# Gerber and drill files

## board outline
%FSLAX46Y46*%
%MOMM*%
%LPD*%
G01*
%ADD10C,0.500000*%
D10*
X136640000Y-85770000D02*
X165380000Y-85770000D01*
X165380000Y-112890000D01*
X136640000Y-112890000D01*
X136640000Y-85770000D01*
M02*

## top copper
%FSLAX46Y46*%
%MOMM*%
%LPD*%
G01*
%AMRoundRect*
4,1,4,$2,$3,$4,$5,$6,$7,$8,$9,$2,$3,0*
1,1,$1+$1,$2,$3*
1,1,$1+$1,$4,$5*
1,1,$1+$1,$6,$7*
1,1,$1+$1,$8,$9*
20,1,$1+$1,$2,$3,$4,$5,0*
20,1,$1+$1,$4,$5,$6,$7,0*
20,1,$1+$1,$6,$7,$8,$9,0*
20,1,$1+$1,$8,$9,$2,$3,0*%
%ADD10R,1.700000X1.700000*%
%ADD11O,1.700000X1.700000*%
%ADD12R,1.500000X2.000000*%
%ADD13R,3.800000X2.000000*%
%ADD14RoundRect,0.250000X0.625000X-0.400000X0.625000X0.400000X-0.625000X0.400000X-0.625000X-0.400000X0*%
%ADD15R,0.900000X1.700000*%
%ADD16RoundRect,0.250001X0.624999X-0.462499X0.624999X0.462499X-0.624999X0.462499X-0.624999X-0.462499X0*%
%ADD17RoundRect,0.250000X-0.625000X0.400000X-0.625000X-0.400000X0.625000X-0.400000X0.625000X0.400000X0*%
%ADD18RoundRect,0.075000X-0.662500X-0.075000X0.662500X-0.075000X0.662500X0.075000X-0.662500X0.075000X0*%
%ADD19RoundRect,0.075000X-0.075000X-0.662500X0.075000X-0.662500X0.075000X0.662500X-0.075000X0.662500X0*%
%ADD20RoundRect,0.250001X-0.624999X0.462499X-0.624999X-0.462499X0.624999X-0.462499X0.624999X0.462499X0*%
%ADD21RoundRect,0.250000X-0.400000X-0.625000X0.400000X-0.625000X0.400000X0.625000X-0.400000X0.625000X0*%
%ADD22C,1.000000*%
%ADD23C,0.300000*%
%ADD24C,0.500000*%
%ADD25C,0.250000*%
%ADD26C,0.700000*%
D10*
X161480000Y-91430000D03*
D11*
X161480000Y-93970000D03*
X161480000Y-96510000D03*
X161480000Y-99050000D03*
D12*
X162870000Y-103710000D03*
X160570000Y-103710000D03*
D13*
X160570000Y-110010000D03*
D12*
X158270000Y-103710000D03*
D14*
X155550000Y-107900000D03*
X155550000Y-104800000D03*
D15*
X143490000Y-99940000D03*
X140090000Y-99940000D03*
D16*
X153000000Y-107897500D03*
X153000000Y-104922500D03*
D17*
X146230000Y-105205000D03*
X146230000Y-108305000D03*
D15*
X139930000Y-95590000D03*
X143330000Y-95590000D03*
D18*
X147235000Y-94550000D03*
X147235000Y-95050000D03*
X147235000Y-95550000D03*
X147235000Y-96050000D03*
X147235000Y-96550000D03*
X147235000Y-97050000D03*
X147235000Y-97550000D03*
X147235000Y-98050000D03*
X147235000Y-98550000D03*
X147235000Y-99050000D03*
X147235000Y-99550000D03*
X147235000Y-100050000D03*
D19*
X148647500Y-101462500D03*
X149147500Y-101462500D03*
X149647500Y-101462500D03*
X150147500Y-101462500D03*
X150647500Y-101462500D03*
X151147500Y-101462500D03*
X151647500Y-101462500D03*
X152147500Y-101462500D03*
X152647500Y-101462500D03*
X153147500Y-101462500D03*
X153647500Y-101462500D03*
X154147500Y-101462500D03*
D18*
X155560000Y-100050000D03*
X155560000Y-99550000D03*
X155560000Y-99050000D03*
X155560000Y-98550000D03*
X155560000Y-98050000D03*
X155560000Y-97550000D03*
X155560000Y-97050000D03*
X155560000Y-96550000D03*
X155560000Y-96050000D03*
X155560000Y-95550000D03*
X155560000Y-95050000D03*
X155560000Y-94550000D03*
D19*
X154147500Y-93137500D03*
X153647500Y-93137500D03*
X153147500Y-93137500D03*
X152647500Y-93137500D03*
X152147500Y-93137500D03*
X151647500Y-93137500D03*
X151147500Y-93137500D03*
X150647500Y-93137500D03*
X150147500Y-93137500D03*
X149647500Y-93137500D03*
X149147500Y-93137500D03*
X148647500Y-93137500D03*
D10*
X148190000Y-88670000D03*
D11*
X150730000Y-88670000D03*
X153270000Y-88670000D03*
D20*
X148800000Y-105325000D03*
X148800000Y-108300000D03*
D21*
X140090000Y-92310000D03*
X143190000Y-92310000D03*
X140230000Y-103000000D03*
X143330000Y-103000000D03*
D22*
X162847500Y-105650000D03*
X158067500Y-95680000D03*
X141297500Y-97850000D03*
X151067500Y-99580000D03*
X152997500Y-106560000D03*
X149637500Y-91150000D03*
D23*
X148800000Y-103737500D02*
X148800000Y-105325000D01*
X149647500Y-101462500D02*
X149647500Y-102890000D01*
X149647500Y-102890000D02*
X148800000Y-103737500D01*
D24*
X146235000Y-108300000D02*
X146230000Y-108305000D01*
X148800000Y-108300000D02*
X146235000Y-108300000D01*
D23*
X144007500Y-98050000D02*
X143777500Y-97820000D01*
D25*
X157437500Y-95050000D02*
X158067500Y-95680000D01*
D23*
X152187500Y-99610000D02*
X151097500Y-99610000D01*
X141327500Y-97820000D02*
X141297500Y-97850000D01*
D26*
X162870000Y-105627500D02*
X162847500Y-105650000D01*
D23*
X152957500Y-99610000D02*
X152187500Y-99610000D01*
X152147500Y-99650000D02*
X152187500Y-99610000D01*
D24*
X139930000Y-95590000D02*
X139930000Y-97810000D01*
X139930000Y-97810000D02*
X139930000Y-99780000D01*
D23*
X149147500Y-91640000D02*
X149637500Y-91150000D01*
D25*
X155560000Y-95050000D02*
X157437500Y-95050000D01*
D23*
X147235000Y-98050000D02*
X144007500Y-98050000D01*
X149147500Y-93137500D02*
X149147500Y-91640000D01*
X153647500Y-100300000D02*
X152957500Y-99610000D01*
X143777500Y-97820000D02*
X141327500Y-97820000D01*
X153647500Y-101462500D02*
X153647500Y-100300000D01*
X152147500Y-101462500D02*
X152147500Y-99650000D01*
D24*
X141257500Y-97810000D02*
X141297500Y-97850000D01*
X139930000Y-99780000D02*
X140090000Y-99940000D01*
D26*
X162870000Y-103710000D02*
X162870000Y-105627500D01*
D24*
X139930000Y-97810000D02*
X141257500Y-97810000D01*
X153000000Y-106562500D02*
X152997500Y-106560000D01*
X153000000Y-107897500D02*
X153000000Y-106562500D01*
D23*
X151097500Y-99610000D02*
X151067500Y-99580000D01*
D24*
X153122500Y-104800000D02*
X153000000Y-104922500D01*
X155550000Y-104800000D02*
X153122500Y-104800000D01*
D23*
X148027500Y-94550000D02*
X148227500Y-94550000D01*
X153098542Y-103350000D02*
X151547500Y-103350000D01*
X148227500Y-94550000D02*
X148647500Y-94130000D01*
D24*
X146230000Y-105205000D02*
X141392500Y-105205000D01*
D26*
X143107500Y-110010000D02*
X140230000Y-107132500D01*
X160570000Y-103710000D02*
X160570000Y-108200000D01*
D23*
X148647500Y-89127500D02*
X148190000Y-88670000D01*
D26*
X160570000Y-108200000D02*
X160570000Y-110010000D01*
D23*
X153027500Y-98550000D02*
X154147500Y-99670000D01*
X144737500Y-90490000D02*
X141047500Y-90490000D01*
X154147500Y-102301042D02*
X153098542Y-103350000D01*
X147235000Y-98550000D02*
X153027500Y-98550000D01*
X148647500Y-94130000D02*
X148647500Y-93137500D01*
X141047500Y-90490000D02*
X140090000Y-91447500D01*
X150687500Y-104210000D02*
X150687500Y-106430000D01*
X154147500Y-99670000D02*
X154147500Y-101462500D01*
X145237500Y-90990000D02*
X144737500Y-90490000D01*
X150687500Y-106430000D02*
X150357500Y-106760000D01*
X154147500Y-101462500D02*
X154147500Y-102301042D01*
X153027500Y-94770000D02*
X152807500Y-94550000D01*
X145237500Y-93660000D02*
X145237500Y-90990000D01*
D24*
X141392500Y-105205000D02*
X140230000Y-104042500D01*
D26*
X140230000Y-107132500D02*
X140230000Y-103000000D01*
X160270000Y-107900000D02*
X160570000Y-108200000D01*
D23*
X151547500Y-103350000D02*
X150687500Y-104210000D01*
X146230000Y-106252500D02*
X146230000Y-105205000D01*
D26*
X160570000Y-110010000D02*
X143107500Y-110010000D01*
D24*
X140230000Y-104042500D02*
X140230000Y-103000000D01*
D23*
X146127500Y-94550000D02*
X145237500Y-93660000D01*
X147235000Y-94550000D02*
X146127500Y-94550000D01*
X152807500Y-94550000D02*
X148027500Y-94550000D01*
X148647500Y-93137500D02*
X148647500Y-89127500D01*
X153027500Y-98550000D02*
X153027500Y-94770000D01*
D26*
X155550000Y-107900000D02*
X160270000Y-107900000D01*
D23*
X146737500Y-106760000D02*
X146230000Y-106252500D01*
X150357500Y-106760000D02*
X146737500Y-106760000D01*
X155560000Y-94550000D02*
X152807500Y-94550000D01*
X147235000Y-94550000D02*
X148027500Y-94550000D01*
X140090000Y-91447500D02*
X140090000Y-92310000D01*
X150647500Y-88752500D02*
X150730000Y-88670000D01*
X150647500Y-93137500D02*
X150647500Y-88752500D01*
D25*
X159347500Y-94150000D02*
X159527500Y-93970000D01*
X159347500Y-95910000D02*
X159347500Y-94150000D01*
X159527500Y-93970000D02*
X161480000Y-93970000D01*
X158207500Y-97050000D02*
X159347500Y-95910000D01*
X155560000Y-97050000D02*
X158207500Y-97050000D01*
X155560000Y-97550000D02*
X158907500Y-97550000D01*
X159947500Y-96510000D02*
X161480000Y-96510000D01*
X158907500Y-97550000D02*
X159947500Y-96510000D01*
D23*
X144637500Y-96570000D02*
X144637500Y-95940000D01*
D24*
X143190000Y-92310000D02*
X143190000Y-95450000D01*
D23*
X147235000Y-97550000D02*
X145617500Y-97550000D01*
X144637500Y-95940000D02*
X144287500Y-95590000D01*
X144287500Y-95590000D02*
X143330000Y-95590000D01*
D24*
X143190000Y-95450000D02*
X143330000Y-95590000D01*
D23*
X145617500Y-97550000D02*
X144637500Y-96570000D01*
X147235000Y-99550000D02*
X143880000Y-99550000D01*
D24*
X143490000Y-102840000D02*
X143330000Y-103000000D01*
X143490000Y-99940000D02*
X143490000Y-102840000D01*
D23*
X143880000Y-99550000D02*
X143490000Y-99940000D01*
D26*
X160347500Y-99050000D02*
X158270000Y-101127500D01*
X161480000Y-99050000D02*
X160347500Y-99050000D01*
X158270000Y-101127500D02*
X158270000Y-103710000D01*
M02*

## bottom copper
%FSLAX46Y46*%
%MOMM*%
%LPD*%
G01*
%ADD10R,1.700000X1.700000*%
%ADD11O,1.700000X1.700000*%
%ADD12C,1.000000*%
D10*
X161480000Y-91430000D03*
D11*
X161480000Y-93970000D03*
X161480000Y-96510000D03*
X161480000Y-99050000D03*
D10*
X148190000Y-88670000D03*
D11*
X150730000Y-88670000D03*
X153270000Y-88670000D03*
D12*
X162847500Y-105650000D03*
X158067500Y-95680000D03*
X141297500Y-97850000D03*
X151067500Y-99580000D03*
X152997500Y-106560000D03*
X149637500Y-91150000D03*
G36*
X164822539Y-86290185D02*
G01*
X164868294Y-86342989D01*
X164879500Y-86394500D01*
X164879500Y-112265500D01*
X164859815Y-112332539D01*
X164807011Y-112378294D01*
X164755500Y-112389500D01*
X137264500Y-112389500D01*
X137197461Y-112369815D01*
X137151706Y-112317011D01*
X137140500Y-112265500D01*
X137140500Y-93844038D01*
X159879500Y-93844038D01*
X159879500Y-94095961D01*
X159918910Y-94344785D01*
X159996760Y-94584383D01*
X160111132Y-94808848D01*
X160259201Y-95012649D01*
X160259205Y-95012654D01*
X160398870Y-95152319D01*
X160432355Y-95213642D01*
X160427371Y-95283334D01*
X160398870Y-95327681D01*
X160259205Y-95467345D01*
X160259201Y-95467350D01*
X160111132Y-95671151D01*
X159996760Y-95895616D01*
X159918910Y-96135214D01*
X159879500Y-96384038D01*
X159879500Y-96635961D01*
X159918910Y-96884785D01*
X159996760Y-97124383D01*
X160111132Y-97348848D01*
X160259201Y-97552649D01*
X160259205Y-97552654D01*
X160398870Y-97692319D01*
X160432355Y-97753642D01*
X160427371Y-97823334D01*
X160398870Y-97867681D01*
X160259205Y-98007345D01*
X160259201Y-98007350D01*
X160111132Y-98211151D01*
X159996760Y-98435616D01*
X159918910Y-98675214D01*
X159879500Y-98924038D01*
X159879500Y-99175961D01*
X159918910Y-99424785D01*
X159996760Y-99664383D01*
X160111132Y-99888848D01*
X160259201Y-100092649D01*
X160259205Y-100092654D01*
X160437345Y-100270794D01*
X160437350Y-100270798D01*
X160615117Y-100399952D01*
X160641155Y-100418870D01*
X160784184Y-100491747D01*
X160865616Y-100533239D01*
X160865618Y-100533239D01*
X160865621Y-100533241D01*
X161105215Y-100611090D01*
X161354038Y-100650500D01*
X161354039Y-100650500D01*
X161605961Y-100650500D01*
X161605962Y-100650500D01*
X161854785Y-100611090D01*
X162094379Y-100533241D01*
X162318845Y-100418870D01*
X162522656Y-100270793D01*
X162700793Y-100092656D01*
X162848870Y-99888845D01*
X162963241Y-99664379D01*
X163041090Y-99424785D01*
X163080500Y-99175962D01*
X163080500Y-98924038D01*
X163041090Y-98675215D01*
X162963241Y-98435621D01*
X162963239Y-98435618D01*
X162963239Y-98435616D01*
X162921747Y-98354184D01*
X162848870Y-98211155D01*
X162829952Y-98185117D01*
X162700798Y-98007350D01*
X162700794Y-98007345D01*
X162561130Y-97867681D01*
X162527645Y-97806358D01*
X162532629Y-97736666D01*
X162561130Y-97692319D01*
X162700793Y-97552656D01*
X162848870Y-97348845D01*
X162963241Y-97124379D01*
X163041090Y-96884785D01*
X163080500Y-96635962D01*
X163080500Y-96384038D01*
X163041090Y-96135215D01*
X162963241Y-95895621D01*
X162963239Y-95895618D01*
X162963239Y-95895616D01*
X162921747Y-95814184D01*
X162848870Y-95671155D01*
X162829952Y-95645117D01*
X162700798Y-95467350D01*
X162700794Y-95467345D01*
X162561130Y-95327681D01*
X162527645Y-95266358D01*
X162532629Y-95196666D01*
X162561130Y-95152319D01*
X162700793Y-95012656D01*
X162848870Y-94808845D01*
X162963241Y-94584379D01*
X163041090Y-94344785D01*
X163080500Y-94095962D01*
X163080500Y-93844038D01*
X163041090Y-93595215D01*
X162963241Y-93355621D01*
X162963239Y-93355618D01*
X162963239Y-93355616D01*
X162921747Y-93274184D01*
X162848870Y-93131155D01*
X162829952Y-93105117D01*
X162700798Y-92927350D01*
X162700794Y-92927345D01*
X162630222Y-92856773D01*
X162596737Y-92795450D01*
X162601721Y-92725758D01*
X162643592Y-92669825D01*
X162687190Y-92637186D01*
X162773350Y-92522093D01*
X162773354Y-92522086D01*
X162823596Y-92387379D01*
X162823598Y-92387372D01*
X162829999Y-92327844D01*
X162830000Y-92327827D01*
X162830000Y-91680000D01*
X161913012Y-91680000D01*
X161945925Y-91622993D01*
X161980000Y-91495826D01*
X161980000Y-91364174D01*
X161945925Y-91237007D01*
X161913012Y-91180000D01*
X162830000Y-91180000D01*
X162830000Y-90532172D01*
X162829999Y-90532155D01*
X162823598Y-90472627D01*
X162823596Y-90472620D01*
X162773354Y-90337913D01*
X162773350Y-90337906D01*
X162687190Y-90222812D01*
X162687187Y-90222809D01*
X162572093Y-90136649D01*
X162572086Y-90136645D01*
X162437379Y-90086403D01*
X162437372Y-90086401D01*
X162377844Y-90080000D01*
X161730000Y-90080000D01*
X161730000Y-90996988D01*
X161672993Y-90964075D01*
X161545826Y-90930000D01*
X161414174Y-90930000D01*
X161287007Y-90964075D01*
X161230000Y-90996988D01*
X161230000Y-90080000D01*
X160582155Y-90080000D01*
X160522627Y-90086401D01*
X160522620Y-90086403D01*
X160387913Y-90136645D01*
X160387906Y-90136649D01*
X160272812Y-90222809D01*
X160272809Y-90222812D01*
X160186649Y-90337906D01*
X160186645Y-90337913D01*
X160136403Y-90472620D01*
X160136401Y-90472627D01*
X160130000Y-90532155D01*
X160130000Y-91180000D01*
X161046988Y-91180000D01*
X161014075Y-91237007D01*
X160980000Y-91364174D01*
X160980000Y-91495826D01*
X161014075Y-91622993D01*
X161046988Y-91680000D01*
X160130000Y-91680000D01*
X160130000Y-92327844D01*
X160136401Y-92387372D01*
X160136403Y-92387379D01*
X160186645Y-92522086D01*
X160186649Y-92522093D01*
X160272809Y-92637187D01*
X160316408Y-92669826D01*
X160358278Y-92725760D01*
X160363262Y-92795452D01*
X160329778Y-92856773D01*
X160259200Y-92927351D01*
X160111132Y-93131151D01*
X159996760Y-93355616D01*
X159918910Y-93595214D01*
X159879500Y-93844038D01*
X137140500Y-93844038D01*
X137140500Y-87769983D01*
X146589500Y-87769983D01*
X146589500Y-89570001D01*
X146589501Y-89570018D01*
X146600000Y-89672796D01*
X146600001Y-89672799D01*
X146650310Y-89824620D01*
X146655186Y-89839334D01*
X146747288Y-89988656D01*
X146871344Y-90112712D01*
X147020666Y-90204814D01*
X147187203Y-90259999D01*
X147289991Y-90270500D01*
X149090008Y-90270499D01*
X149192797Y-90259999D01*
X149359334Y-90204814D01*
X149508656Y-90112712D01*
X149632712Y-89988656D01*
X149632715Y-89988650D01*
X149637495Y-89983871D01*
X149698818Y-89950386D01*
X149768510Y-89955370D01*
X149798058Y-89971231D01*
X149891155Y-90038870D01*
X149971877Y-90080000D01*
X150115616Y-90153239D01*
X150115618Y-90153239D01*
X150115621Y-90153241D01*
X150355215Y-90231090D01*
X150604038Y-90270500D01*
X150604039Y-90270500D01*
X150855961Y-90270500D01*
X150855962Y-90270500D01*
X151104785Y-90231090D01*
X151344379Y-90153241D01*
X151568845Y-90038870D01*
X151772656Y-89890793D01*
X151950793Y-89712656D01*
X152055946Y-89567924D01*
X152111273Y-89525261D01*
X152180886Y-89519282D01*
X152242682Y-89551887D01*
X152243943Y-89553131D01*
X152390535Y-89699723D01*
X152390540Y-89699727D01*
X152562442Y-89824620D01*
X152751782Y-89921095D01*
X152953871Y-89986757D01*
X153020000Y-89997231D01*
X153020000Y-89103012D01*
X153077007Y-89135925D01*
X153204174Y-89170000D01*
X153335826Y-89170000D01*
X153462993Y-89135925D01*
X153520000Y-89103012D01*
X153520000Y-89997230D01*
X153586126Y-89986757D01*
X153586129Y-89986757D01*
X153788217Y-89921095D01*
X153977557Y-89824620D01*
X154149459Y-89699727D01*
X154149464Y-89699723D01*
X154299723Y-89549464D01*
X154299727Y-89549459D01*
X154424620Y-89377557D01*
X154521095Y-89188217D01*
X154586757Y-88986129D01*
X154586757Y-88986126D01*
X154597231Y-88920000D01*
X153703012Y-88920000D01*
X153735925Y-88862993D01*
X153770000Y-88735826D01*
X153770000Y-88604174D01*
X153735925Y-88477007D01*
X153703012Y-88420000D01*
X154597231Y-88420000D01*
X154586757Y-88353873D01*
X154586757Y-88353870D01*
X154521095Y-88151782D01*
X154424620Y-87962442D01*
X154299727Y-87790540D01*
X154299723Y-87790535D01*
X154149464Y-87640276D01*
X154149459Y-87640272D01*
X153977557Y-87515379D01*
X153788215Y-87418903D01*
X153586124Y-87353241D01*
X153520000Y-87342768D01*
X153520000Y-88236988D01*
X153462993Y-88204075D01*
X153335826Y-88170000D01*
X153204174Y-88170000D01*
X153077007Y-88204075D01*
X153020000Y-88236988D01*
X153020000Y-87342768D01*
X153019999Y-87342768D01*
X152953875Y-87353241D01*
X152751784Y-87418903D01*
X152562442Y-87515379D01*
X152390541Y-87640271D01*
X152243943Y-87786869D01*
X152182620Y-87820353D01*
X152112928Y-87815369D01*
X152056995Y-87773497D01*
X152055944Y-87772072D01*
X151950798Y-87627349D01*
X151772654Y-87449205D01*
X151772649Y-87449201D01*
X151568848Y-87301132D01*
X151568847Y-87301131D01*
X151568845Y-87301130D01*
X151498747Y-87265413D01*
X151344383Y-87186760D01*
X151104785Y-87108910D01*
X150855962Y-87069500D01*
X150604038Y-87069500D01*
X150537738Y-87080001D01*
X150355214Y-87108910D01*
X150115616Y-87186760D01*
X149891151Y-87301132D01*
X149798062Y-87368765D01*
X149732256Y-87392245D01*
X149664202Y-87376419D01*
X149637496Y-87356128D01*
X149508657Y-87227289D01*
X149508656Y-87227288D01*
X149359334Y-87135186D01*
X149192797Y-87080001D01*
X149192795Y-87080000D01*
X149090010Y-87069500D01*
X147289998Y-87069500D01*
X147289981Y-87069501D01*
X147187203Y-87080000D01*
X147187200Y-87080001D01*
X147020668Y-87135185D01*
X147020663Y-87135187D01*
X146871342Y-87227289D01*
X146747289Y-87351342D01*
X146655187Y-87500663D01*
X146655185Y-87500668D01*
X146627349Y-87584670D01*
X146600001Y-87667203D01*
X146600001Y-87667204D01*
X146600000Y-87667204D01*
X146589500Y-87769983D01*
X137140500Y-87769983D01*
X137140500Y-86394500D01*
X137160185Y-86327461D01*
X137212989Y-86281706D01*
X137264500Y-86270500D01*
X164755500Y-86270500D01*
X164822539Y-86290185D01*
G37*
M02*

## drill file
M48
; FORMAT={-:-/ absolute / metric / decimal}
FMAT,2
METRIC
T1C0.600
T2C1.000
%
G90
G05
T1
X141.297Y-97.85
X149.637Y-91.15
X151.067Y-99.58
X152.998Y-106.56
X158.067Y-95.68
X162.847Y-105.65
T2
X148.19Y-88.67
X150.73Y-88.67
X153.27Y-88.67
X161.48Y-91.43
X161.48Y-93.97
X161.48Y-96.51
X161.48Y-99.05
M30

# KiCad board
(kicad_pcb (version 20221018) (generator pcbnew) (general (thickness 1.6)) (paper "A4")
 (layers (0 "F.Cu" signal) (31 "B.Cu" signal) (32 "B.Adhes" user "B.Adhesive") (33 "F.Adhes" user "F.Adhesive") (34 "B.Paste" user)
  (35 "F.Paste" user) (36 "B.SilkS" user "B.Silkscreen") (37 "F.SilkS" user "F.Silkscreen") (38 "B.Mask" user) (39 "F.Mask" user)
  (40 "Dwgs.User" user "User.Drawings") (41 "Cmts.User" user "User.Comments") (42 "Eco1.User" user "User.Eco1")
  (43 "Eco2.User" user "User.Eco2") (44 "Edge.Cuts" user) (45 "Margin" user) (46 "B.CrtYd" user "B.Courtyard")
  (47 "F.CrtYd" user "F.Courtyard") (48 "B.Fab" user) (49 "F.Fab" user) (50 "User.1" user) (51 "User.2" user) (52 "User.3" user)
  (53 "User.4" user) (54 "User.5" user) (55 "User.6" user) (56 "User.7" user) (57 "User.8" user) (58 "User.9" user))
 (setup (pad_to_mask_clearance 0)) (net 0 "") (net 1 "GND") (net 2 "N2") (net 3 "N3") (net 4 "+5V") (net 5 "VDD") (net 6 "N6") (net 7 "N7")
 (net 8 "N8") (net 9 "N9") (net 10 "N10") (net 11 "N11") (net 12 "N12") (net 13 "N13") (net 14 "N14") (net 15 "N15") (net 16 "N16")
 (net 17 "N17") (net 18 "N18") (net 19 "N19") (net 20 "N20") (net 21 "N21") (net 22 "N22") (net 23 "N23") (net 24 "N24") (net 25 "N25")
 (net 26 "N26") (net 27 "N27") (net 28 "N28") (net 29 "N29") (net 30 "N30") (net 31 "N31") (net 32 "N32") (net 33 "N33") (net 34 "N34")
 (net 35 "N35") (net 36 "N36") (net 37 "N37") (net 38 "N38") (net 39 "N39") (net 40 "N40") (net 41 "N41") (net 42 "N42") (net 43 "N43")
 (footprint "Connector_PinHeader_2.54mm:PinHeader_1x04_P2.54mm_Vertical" (layer "F.Cu") (at 161.48 91.43)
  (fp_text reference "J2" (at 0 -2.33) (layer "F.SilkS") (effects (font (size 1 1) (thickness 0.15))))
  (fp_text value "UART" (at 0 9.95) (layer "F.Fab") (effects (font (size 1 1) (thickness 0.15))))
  (pad "1" thru_hole rect (at 0 0) (size 1.7 1.7) (drill 1) (layers "*.Cu" "*.Mask") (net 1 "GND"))
  (pad "2" thru_hole oval (at 0 2.54) (size 1.7 1.7) (drill 1) (layers "*.Cu" "*.Mask") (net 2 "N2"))
  (pad "3" thru_hole oval (at 0 5.08) (size 1.7 1.7) (drill 1) (layers "*.Cu" "*.Mask") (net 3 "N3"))
  (pad "4" thru_hole oval (at 0 7.62) (size 1.7 1.7) (drill 1) (layers "*.Cu" "*.Mask") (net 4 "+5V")))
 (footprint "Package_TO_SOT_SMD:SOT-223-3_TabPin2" (layer "F.Cu") (at 160.57 106.86 -90)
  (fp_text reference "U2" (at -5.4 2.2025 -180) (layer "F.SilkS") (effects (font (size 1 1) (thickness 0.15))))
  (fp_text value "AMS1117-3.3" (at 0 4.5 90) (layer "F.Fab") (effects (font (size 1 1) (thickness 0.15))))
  (pad "1" smd rect (at -3.15 -2.3 270) (size 2 1.5) (layers "F.Cu" "F.Paste" "F.Mask") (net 1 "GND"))
  (pad "2" smd rect (at -3.15 0 270) (size 2 1.5) (layers "F.Cu" "F.Paste" "F.Mask") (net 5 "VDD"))
  (pad "2" smd rect (at 3.15 0 270) (size 2 3.8) (layers "F.Cu" "F.Paste" "F.Mask") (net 5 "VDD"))
  (pad "3" smd rect (at -3.15 2.3 270) (size 2 1.5) (layers "F.Cu" "F.Paste" "F.Mask") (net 4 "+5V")))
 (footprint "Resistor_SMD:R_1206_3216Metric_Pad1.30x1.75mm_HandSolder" (layer "F.Cu") (at 155.55 106.35 90)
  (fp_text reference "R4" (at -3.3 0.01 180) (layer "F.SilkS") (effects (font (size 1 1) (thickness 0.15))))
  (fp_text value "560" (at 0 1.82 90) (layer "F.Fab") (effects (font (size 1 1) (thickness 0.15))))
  (pad "1" smd roundrect (at -1.55 0 90) (size 1.3 1.75) (layers "F.Cu" "F.Paste" "F.Mask") (roundrect_rratio 0.1923076923) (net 5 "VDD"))
  (pad "2" smd roundrect (at 1.55 0 90) (size 1.3 1.75) (layers "F.Cu" "F.Paste" "F.Mask") (roundrect_rratio 0.1923076923) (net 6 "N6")))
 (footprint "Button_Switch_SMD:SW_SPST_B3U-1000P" (layer "F.Cu") (at 141.79 99.94 180)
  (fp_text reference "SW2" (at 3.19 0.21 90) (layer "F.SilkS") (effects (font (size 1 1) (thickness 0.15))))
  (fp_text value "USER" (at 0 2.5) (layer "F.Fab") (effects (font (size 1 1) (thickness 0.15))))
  (pad "1" smd rect (at -1.7 0 180) (size 0.9 1.7) (layers "F.Cu" "F.Paste" "F.Mask") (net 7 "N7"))
  (pad "2" smd rect (at 1.7 0 180) (size 0.9 1.7) (layers "F.Cu" "F.Paste" "F.Mask") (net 1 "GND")))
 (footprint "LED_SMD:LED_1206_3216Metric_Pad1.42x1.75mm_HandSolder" (layer "F.Cu") (at 153 106.41 90)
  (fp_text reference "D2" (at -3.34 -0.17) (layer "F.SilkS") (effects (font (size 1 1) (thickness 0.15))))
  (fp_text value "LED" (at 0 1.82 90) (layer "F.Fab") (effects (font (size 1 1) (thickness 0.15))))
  (pad "1" smd roundrect (at -1.4875 0 90) (size 1.425 1.75) (layers "F.Cu" "F.Paste" "F.Mask") (roundrect_rratio 0.1754392982)
   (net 1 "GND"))
  (pad "2" smd roundrect (at 1.4875 0 90) (size 1.425 1.75) (layers "F.Cu" "F.Paste" "F.Mask") (roundrect_rratio 0.1754392982) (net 6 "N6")))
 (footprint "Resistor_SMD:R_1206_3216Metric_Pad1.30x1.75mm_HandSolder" (layer "F.Cu") (at 146.23 106.755 -90)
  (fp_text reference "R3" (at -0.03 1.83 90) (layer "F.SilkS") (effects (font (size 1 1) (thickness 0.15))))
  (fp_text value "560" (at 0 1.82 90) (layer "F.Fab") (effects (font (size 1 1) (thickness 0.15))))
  (pad "1" smd roundrect (at -1.55 0 270) (size 1.3 1.75) (layers "F.Cu" "F.Paste" "F.Mask") (roundrect_rratio 0.1923076923) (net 5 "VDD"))
  (pad "2" smd roundrect (at 1.55 0 270) (size 1.3 1.75) (layers "F.Cu" "F.Paste" "F.Mask") (roundrect_rratio 0.1923076923) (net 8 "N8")))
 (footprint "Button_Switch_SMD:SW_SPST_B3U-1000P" (layer "F.Cu") (at 141.63 95.59)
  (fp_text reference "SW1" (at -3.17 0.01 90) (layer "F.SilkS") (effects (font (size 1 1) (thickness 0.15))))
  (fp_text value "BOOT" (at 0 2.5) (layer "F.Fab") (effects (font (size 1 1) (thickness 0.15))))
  (pad "1" smd rect (at -1.7 0) (size 0.9 1.7) (layers "F.Cu" "F.Paste" "F.Mask") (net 1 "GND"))
  (pad "2" smd rect (at 1.7 0) (size 0.9 1.7) (layers "F.Cu" "F.Paste" "F.Mask") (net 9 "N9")))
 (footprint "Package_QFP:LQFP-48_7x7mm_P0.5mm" (layer "F.Cu") (at 151.3975 97.3)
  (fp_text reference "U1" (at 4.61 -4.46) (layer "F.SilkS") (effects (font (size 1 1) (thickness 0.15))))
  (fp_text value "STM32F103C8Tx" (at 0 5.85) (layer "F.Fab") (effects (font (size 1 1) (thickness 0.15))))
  (pad "1" smd roundrect (at -4.1625 -2.75) (size 1.475 0.3) (layers "F.Cu" "F.Paste" "F.Mask") (roundrect_rratio 0.25) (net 5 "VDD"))
  (pad "2" smd roundrect (at -4.1625 -2.25) (size 1.475 0.3) (layers "F.Cu" "F.Paste" "F.Mask") (roundrect_rratio 0.25) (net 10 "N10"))
  (pad "3" smd roundrect (at -4.1625 -1.75) (size 1.475 0.3) (layers "F.Cu" "F.Paste" "F.Mask") (roundrect_rratio 0.25) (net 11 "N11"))
  (pad "4" smd roundrect (at -4.1625 -1.25) (size 1.475 0.3) (layers "F.Cu" "F.Paste" "F.Mask") (roundrect_rratio 0.25) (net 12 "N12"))
  (pad "5" smd roundrect (at -4.1625 -0.75) (size 1.475 0.3) (layers "F.Cu" "F.Paste" "F.Mask") (roundrect_rratio 0.25) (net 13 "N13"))
  (pad "6" smd roundrect (at -4.1625 -0.25) (size 1.475 0.3) (layers "F.Cu" "F.Paste" "F.Mask") (roundrect_rratio 0.25) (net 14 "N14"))
  (pad "7" smd roundrect (at -4.1625 0.25) (size 1.475 0.3) (layers "F.Cu" "F.Paste" "F.Mask") (roundrect_rratio 0.25) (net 9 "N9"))
  (pad "8" smd roundrect (at -4.1625 0.75) (size 1.475 0.3) (layers "F.Cu" "F.Paste" "F.Mask") (roundrect_rratio 0.25) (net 1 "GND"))
  (pad "9" smd roundrect (at -4.1625 1.25) (size 1.475 0.3) (layers "F.Cu" "F.Paste" "F.Mask") (roundrect_rratio 0.25) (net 5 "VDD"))
  (pad "10" smd roundrect (at -4.1625 1.75) (size 1.475 0.3) (layers "F.Cu" "F.Paste" "F.Mask") (roundrect_rratio 0.25) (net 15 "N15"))
  (pad "11" smd roundrect (at -4.1625 2.25) (size 1.475 0.3) (layers "F.Cu" "F.Paste" "F.Mask") (roundrect_rratio 0.25) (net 7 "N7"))
  (pad "12" smd roundrect (at -4.1625 2.75) (size 1.475 0.3) (layers "F.Cu" "F.Paste" "F.Mask") (roundrect_rratio 0.25) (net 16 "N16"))
  (pad "13" smd roundrect (at -2.75 4.1625) (size 0.3 1.475) (layers "F.Cu" "F.Paste" "F.Mask") (roundrect_rratio 0.25) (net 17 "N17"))
  (pad "14" smd roundrect (at -2.25 4.1625) (size 0.3 1.475) (layers "F.Cu" "F.Paste" "F.Mask") (roundrect_rratio 0.25) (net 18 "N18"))
  (pad "15" smd roundrect (at -1.75 4.1625) (size 0.3 1.475) (layers "F.Cu" "F.Paste" "F.Mask") (roundrect_rratio 0.25) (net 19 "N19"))
  (pad "16" smd roundrect (at -1.25 4.1625) (size 0.3 1.475) (layers "F.Cu" "F.Paste" "F.Mask") (roundrect_rratio 0.25) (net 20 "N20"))
  (pad "17" smd roundrect (at -0.75 4.1625) (size 0.3 1.475) (layers "F.Cu" "F.Paste" "F.Mask") (roundrect_rratio 0.25) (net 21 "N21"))
  (pad "18" smd roundrect (at -0.25 4.1625) (size 0.3 1.475) (layers "F.Cu" "F.Paste" "F.Mask") (roundrect_rratio 0.25) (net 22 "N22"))
  (pad "19" smd roundrect (at 0.25 4.1625) (size 0.3 1.475) (layers "F.Cu" "F.Paste" "F.Mask") (roundrect_rratio 0.25) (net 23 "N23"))
  (pad "20" smd roundrect (at 0.75 4.1625) (size 0.3 1.475) (layers "F.Cu" "F.Paste" "F.Mask") (roundrect_rratio 0.25) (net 1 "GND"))
  (pad "21" smd roundrect (at 1.25 4.1625) (size 0.3 1.475) (layers "F.Cu" "F.Paste" "F.Mask") (roundrect_rratio 0.25) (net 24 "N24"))
  (pad "22" smd roundrect (at 1.75 4.1625) (size 0.3 1.475) (layers "F.Cu" "F.Paste" "F.Mask") (roundrect_rratio 0.25) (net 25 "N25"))
  (pad "23" smd roundrect (at 2.25 4.1625) (size 0.3 1.475) (layers "F.Cu" "F.Paste" "F.Mask") (roundrect_rratio 0.25) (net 1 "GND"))
  (pad "24" smd roundrect (at 2.75 4.1625) (size 0.3 1.475) (layers "F.Cu" "F.Paste" "F.Mask") (roundrect_rratio 0.25) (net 5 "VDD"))
  (pad "25" smd roundrect (at 4.1625 2.75) (size 1.475 0.3) (layers "F.Cu" "F.Paste" "F.Mask") (roundrect_rratio 0.25) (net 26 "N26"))
  (pad "26" smd roundrect (at 4.1625 2.25) (size 1.475 0.3) (layers "F.Cu" "F.Paste" "F.Mask") (roundrect_rratio 0.25) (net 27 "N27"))
  (pad "27" smd roundrect (at 4.1625 1.75) (size 1.475 0.3) (layers "F.Cu" "F.Paste" "F.Mask") (roundrect_rratio 0.25) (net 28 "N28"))
  (pad "28" smd roundrect (at 4.1625 1.25) (size 1.475 0.3) (layers "F.Cu" "F.Paste" "F.Mask") (roundrect_rratio 0.25) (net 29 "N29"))
  (pad "29" smd roundrect (at 4.1625 0.75) (size 1.475 0.3) (layers "F.Cu" "F.Paste" "F.Mask") (roundrect_rratio 0.25) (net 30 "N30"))
  (pad "30" smd roundrect (at 4.1625 0.25) (size 1.475 0.3) (layers "F.Cu" "F.Paste" "F.Mask") (roundrect_rratio 0.25) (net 3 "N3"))
  (pad "31" smd roundrect (at 4.1625 -0.25) (size 1.475 0.3) (layers "F.Cu" "F.Paste" "F.Mask") (roundrect_rratio 0.25) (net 2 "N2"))
  (pad "32" smd roundrect (at 4.1625 -0.75) (size 1.475 0.3) (layers "F.Cu" "F.Paste" "F.Mask") (roundrect_rratio 0.25) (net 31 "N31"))
  (pad "33" smd roundrect (at 4.1625 -1.25) (size 1.475 0.3) (layers "F.Cu" "F.Paste" "F.Mask") (roundrect_rratio 0.25) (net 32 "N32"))
  (pad "34" smd roundrect (at 4.1625 -1.75) (size 1.475 0.3) (layers "F.Cu" "F.Paste" "F.Mask") (roundrect_rratio 0.25) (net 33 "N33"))
  (pad "35" smd roundrect (at 4.1625 -2.25) (size 1.475 0.3) (layers "F.Cu" "F.Paste" "F.Mask") (roundrect_rratio 0.25) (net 1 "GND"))
  (pad "36" smd roundrect (at 4.1625 -2.75) (size 1.475 0.3) (layers "F.Cu" "F.Paste" "F.Mask") (roundrect_rratio 0.25) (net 5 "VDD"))
  (pad "37" smd roundrect (at 2.75 -4.1625) (size 0.3 1.475) (layers "F.Cu" "F.Paste" "F.Mask") (roundrect_rratio 0.25) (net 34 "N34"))
  (pad "38" smd roundrect (at 2.25 -4.1625) (size 0.3 1.475) (layers "F.Cu" "F.Paste" "F.Mask") (roundrect_rratio 0.25) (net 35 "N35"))
  (pad "39" smd roundrect (at 1.75 -4.1625) (size 0.3 1.475) (layers "F.Cu" "F.Paste" "F.Mask") (roundrect_rratio 0.25) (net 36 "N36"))
  (pad "40" smd roundrect (at 1.25 -4.1625) (size 0.3 1.475) (layers "F.Cu" "F.Paste" "F.Mask") (roundrect_rratio 0.25) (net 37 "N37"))
  (pad "41" smd roundrect (at 0.75 -4.1625) (size 0.3 1.475) (layers "F.Cu" "F.Paste" "F.Mask") (roundrect_rratio 0.25) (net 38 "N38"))
  (pad "42" smd roundrect (at 0.25 -4.1625) (size 0.3 1.475) (layers "F.Cu" "F.Paste" "F.Mask") (roundrect_rratio 0.25) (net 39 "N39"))
  (pad "43" smd roundrect (at -0.25 -4.1625) (size 0.3 1.475) (layers "F.Cu" "F.Paste" "F.Mask") (roundrect_rratio 0.25) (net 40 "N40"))
  (pad "44" smd roundrect (at -0.75 -4.1625) (size 0.3 1.475) (layers "F.Cu" "F.Paste" "F.Mask") (roundrect_rratio 0.25) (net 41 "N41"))
  (pad "45" smd roundrect (at -1.25 -4.1625) (size 0.3 1.475) (layers "F.Cu" "F.Paste" "F.Mask") (roundrect_rratio 0.25) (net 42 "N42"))
  (pad "46" smd roundrect (at -1.75 -4.1625) (size 0.3 1.475) (layers "F.Cu" "F.Paste" "F.Mask") (roundrect_rratio 0.25) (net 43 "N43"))
  (pad "47" smd roundrect (at -2.25 -4.1625) (size 0.3 1.475) (layers "F.Cu" "F.Paste" "F.Mask") (roundrect_rratio 0.25) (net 1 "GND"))
  (pad "48" smd roundrect (at -2.75 -4.1625) (size 0.3 1.475) (layers "F.Cu" "F.Paste" "F.Mask") (roundrect_rratio 0.25) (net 5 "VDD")))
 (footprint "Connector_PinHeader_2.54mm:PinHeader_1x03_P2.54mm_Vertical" (layer "F.Cu") (at 148.19 88.67 90)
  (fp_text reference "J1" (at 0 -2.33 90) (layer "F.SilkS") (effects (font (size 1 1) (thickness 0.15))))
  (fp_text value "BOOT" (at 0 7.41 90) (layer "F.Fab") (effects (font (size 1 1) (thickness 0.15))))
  (pad "1" thru_hole rect (at 0 0 90) (size 1.7 1.7) (drill 1) (layers "*.Cu" "*.Mask") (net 5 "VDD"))
  (pad "2" thru_hole oval (at 0 2.54 90) (size 1.7 1.7) (drill 1) (layers "*.Cu" "*.Mask") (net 41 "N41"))
  (pad "3" thru_hole oval (at 0 5.08 90) (size 1.7 1.7) (drill 1) (layers "*.Cu" "*.Mask") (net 1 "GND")))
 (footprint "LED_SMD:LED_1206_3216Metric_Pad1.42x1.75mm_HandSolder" (layer "F.Cu") (at 148.8 106.8125 -90)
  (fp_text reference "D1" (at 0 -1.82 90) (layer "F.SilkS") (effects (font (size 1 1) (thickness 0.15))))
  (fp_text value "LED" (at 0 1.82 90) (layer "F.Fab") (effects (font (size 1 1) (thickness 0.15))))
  (pad "1" smd roundrect (at -1.4875 0 270) (size 1.425 1.75) (layers "F.Cu" "F.Paste" "F.Mask") (roundrect_rratio 0.1754392982)
   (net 19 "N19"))
  (pad "2" smd roundrect (at 1.4875 0 270) (size 1.425 1.75) (layers "F.Cu" "F.Paste" "F.Mask") (roundrect_rratio 0.1754392982) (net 8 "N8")))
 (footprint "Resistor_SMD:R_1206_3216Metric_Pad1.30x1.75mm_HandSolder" (layer "F.Cu") (at 141.64 92.31)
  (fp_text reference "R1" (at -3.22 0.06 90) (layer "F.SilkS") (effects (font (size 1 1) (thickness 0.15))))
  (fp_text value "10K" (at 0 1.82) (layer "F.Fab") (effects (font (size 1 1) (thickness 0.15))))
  (pad "1" smd roundrect (at -1.55 0) (size 1.3 1.75) (layers "F.Cu" "F.Paste" "F.Mask") (roundrect_rratio 0.1923076923) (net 5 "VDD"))
  (pad "2" smd roundrect (at 1.55 0) (size 1.3 1.75) (layers "F.Cu" "F.Paste" "F.Mask") (roundrect_rratio 0.1923076923) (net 9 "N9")))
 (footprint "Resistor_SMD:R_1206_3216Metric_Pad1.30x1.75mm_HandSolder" (layer "F.Cu") (at 141.78 103)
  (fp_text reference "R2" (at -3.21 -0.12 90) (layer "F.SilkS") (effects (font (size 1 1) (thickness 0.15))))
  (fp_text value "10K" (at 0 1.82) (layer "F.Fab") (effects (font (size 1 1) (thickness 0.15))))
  (pad "1" smd roundrect (at -1.55 0) (size 1.3 1.75) (layers "F.Cu" "F.Paste" "F.Mask") (roundrect_rratio 0.1923076923) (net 5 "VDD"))
  (pad "2" smd roundrect (at 1.55 0) (size 1.3 1.75) (layers "F.Cu" "F.Paste" "F.Mask") (roundrect_rratio 0.1923076923) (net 7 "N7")))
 (gr_rect (start 136.64 85.77) (end 165.38 112.89) (stroke (width 0.5) (type default)) (fill none) (layer "Edge.Cuts"))
 (segment (start 148.8 103.7375) (end 148.8 105.325) (width 0.3) (layer "F.Cu") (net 19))
 (segment (start 149.6475 101.4625) (end 149.6475 102.89) (width 0.3) (layer "F.Cu") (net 19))
 (segment (start 149.6475 102.89) (end 148.8 103.7375) (width 0.3) (layer "F.Cu") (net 19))
 (segment (start 146.235 108.3) (end 146.23 108.305) (width 0.5) (layer "F.Cu") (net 8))
 (segment (start 148.8 108.3) (end 146.235 108.3) (width 0.5) (layer "F.Cu") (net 8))
 (segment (start 144.0075 98.05) (end 143.7775 97.82) (width 0.3) (layer "F.Cu") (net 1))
 (segment (start 157.4375 95.05) (end 158.0675 95.68) (width 0.25) (layer "F.Cu") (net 1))
 (segment (start 152.1875 99.61) (end 151.0975 99.61) (width 0.3) (layer "F.Cu") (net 1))
 (segment (start 141.3275 97.82) (end 141.2975 97.85) (width 0.3) (layer "F.Cu") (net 1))
 (segment (start 162.87 105.6275) (end 162.8475 105.65) (width 0.7) (layer "F.Cu") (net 1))
 (segment (start 152.9575 99.61) (end 152.1875 99.61) (width 0.3) (layer "F.Cu") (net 1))
 (segment (start 152.1475 99.65) (end 152.1875 99.61) (width 0.3) (layer "F.Cu") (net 1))
 (segment (start 139.93 95.59) (end 139.93 97.81) (width 0.5) (layer "F.Cu") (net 1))
 (segment (start 139.93 97.81) (end 139.93 99.78) (width 0.5) (layer "F.Cu") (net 1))
 (segment (start 149.1475 91.64) (end 149.6375 91.15) (width 0.3) (layer "F.Cu") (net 1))
 (segment (start 155.56 95.05) (end 157.4375 95.05) (width 0.25) (layer "F.Cu") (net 1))
 (segment (start 147.235 98.05) (end 144.0075 98.05) (width 0.3) (layer "F.Cu") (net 1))
 (segment (start 149.1475 93.1375) (end 149.1475 91.64) (width 0.3) (layer "F.Cu") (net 1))
 (segment (start 153.6475 100.3) (end 152.9575 99.61) (width 0.3) (layer "F.Cu") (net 1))
 (segment (start 143.7775 97.82) (end 141.3275 97.82) (width 0.3) (layer "F.Cu") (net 1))
 (segment (start 153.6475 101.4625) (end 153.6475 100.3) (width 0.3) (layer "F.Cu") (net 1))
 (segment (start 152.1475 101.4625) (end 152.1475 99.65) (width 0.3) (layer "F.Cu") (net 1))
 (segment (start 141.2575 97.81) (end 141.2975 97.85) (width 0.5) (layer "F.Cu") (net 1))
 (segment (start 139.93 99.78) (end 140.09 99.94) (width 0.5) (layer "F.Cu") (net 1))
 (segment (start 162.87 103.71) (end 162.87 105.6275) (width 0.7) (layer "F.Cu") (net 1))
 (segment (start 139.93 97.81) (end 141.2575 97.81) (width 0.5) (layer "F.Cu") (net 1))
 (segment (start 153 106.5625) (end 152.9975 106.56) (width 0.5) (layer "F.Cu") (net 1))
 (segment (start 153 107.8975) (end 153 106.5625) (width 0.5) (layer "F.Cu") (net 1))
 (segment (start 151.0975 99.61) (end 151.0675 99.58) (width 0.3) (layer "F.Cu") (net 1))
 (via (at 162.8475 105.65) (size 1) (drill 0.6) (layers "F.Cu" "B.Cu") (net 1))
 (via (at 158.0675 95.68) (size 1) (drill 0.6) (layers "F.Cu" "B.Cu") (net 1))
 (via (at 141.2975 97.85) (size 1) (drill 0.6) (layers "F.Cu" "B.Cu") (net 1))
 (via (at 151.0675 99.58) (size 1) (drill 0.6) (layers "F.Cu" "B.Cu") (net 1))
 (via (at 152.9975 106.56) (size 1) (drill 0.6) (layers "F.Cu" "B.Cu") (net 1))
 (via (at 149.6375 91.15) (size 1) (drill 0.6) (layers "F.Cu" "B.Cu") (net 1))
 (segment (start 153.1225 104.8) (end 153 104.9225) (width 0.5) (layer "F.Cu") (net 6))
 (segment (start 155.55 104.8) (end 153.1225 104.8) (width 0.5) (layer "F.Cu") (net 6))
 (segment (start 148.0275 94.55) (end 148.2275 94.55) (width 0.3) (layer "F.Cu") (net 5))
 (segment (start 153.098542 103.35) (end 151.5475 103.35) (width 0.3) (layer "F.Cu") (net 5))
 (segment (start 148.2275 94.55) (end 148.6475 94.13) (width 0.3) (layer "F.Cu") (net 5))
 (segment (start 146.23 105.205) (end 141.3925 105.205) (width 0.5) (layer "F.Cu") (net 5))
 (segment (start 143.1075 110.01) (end 140.23 107.1325) (width 0.7) (layer "F.Cu") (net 5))
 (segment (start 160.57 103.71) (end 160.57 108.2) (width 0.7) (layer "F.Cu") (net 5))
 (segment (start 148.6475 89.1275) (end 148.19 88.67) (width 0.3) (layer "F.Cu") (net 5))
 (segment (start 160.57 108.2) (end 160.57 110.01) (width 0.7) (layer "F.Cu") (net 5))
 (segment (start 153.0275 98.55) (end 154.1475 99.67) (width 0.3) (layer "F.Cu") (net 5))
 (segment (start 144.7375 90.49) (end 141.0475 90.49) (width 0.3) (layer "F.Cu") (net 5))
 (segment (start 154.1475 102.301042) (end 153.098542 103.35) (width 0.3) (layer "F.Cu") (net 5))
 (segment (start 147.235 98.55) (end 153.0275 98.55) (width 0.3) (layer "F.Cu") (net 5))
 (segment (start 148.6475 94.13) (end 148.6475 93.1375) (width 0.3) (layer "F.Cu") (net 5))
 (segment (start 141.0475 90.49) (end 140.09 91.4475) (width 0.3) (layer "F.Cu") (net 5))
 (segment (start 150.6875 104.21) (end 150.6875 106.43) (width 0.3) (layer "F.Cu") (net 5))
 (segment (start 154.1475 99.67) (end 154.1475 101.4625) (width 0.3) (layer "F.Cu") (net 5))
 (segment (start 145.2375 90.99) (end 144.7375 90.49) (width 0.3) (layer "F.Cu") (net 5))
 (segment (start 150.6875 106.43) (end 150.3575 106.76) (width 0.3) (layer "F.Cu") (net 5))
 (segment (start 154.1475 101.4625) (end 154.1475 102.301042) (width 0.3) (layer "F.Cu") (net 5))
 (segment (start 153.0275 94.77) (end 152.8075 94.55) (width 0.3) (layer "F.Cu") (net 5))
 (segment (start 145.2375 93.66) (end 145.2375 90.99) (width 0.3) (layer "F.Cu") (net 5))
 (segment (start 141.3925 105.205) (end 140.23 104.0425) (width 0.5) (layer "F.Cu") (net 5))
 (segment (start 140.23 107.1325) (end 140.23 103) (width 0.7) (layer "F.Cu") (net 5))
 (segment (start 160.27 107.9) (end 160.57 108.2) (width 0.7) (layer "F.Cu") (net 5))
 (segment (start 151.5475 103.35) (end 150.6875 104.21) (width 0.3) (layer "F.Cu") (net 5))
 (segment (start 146.23 106.2525) (end 146.23 105.205) (width 0.3) (layer "F.Cu") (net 5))
 (segment (start 160.57 110.01) (end 143.1075 110.01) (width 0.7) (layer "F.Cu") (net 5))
 (segment (start 140.23 104.0425) (end 140.23 103) (width 0.5) (layer "F.Cu") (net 5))
 (segment (start 146.1275 94.55) (end 145.2375 93.66) (width 0.3) (layer "F.Cu") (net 5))
 (segment (start 147.235 94.55) (end 146.1275 94.55) (width 0.3) (layer "F.Cu") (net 5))
 (segment (start 152.8075 94.55) (end 148.0275 94.55) (width 0.3) (layer "F.Cu") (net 5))
 (segment (start 148.6475 93.1375) (end 148.6475 89.1275) (width 0.3) (layer "F.Cu") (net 5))
 (segment (start 153.0275 98.55) (end 153.0275 94.77) (width 0.3) (layer "F.Cu") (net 5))
 (segment (start 155.55 107.9) (end 160.27 107.9) (width 0.7) (layer "F.Cu") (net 5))
 (segment (start 146.7375 106.76) (end 146.23 106.2525) (width 0.3) (layer "F.Cu") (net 5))
 (segment (start 150.3575 106.76) (end 146.7375 106.76) (width 0.3) (layer "F.Cu") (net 5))
 (segment (start 155.56 94.55) (end 152.8075 94.55) (width 0.3) (layer "F.Cu") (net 5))
 (segment (start 147.235 94.55) (end 148.0275 94.55) (width 0.3) (layer "F.Cu") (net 5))
 (segment (start 140.09 91.4475) (end 140.09 92.31) (width 0.3) (layer "F.Cu") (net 5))
 (segment (start 150.6475 88.7525) (end 150.73 88.67) (width 0.3) (layer "F.Cu") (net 41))
 (segment (start 150.6475 93.1375) (end 150.6475 88.7525) (width 0.3) (layer "F.Cu") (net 41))
 (segment (start 159.3475 94.15) (end 159.5275 93.97) (width 0.25) (layer "F.Cu") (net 2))
 (segment (start 159.3475 95.91) (end 159.3475 94.15) (width 0.25) (layer "F.Cu") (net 2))
 (segment (start 159.5275 93.97) (end 161.48 93.97) (width 0.25) (layer "F.Cu") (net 2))
 (segment (start 158.2075 97.05) (end 159.3475 95.91) (width 0.25) (layer "F.Cu") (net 2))
 (segment (start 155.56 97.05) (end 158.2075 97.05) (width 0.25) (layer "F.Cu") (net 2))
 (segment (start 155.56 97.55) (end 158.9075 97.55) (width 0.25) (layer "F.Cu") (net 3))
 (segment (start 159.9475 96.51) (end 161.48 96.51) (width 0.25) (layer "F.Cu") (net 3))
 (segment (start 158.9075 97.55) (end 159.9475 96.51) (width 0.25) (layer "F.Cu") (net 3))
 (segment (start 144.6375 96.57) (end 144.6375 95.94) (width 0.3) (layer "F.Cu") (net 9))
 (segment (start 143.19 92.31) (end 143.19 95.45) (width 0.5) (layer "F.Cu") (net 9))
 (segment (start 147.235 97.55) (end 145.6175 97.55) (width 0.3) (layer "F.Cu") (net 9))
 (segment (start 144.6375 95.94) (end 144.2875 95.59) (width 0.3) (layer "F.Cu") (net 9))
 (segment (start 144.2875 95.59) (end 143.33 95.59) (width 0.3) (layer "F.Cu") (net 9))
 (segment (start 143.19 95.45) (end 143.33 95.59) (width 0.5) (layer "F.Cu") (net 9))
 (segment (start 145.6175 97.55) (end 144.6375 96.57) (width 0.3) (layer "F.Cu") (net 9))
 (segment (start 147.235 99.55) (end 143.88 99.55) (width 0.3) (layer "F.Cu") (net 7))
 (segment (start 143.49 102.84) (end 143.33 103) (width 0.5) (layer "F.Cu") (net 7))
 (segment (start 143.49 99.94) (end 143.49 102.84) (width 0.5) (layer "F.Cu") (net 7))
 (segment (start 143.88 99.55) (end 143.49 99.94) (width 0.3) (layer "F.Cu") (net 7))
 (segment (start 160.3475 99.05) (end 158.27 101.1275) (width 0.7) (layer "F.Cu") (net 4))
 (segment (start 161.48 99.05) (end 160.3475 99.05) (width 0.7) (layer "F.Cu") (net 4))
 (segment (start 158.27 101.1275) (end 158.27 103.71) (width 0.7) (layer "F.Cu") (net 4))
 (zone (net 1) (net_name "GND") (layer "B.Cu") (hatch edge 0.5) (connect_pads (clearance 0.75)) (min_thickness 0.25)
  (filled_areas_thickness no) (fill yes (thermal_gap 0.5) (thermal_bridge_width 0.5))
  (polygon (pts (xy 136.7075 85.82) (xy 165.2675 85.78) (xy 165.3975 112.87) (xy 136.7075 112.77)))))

